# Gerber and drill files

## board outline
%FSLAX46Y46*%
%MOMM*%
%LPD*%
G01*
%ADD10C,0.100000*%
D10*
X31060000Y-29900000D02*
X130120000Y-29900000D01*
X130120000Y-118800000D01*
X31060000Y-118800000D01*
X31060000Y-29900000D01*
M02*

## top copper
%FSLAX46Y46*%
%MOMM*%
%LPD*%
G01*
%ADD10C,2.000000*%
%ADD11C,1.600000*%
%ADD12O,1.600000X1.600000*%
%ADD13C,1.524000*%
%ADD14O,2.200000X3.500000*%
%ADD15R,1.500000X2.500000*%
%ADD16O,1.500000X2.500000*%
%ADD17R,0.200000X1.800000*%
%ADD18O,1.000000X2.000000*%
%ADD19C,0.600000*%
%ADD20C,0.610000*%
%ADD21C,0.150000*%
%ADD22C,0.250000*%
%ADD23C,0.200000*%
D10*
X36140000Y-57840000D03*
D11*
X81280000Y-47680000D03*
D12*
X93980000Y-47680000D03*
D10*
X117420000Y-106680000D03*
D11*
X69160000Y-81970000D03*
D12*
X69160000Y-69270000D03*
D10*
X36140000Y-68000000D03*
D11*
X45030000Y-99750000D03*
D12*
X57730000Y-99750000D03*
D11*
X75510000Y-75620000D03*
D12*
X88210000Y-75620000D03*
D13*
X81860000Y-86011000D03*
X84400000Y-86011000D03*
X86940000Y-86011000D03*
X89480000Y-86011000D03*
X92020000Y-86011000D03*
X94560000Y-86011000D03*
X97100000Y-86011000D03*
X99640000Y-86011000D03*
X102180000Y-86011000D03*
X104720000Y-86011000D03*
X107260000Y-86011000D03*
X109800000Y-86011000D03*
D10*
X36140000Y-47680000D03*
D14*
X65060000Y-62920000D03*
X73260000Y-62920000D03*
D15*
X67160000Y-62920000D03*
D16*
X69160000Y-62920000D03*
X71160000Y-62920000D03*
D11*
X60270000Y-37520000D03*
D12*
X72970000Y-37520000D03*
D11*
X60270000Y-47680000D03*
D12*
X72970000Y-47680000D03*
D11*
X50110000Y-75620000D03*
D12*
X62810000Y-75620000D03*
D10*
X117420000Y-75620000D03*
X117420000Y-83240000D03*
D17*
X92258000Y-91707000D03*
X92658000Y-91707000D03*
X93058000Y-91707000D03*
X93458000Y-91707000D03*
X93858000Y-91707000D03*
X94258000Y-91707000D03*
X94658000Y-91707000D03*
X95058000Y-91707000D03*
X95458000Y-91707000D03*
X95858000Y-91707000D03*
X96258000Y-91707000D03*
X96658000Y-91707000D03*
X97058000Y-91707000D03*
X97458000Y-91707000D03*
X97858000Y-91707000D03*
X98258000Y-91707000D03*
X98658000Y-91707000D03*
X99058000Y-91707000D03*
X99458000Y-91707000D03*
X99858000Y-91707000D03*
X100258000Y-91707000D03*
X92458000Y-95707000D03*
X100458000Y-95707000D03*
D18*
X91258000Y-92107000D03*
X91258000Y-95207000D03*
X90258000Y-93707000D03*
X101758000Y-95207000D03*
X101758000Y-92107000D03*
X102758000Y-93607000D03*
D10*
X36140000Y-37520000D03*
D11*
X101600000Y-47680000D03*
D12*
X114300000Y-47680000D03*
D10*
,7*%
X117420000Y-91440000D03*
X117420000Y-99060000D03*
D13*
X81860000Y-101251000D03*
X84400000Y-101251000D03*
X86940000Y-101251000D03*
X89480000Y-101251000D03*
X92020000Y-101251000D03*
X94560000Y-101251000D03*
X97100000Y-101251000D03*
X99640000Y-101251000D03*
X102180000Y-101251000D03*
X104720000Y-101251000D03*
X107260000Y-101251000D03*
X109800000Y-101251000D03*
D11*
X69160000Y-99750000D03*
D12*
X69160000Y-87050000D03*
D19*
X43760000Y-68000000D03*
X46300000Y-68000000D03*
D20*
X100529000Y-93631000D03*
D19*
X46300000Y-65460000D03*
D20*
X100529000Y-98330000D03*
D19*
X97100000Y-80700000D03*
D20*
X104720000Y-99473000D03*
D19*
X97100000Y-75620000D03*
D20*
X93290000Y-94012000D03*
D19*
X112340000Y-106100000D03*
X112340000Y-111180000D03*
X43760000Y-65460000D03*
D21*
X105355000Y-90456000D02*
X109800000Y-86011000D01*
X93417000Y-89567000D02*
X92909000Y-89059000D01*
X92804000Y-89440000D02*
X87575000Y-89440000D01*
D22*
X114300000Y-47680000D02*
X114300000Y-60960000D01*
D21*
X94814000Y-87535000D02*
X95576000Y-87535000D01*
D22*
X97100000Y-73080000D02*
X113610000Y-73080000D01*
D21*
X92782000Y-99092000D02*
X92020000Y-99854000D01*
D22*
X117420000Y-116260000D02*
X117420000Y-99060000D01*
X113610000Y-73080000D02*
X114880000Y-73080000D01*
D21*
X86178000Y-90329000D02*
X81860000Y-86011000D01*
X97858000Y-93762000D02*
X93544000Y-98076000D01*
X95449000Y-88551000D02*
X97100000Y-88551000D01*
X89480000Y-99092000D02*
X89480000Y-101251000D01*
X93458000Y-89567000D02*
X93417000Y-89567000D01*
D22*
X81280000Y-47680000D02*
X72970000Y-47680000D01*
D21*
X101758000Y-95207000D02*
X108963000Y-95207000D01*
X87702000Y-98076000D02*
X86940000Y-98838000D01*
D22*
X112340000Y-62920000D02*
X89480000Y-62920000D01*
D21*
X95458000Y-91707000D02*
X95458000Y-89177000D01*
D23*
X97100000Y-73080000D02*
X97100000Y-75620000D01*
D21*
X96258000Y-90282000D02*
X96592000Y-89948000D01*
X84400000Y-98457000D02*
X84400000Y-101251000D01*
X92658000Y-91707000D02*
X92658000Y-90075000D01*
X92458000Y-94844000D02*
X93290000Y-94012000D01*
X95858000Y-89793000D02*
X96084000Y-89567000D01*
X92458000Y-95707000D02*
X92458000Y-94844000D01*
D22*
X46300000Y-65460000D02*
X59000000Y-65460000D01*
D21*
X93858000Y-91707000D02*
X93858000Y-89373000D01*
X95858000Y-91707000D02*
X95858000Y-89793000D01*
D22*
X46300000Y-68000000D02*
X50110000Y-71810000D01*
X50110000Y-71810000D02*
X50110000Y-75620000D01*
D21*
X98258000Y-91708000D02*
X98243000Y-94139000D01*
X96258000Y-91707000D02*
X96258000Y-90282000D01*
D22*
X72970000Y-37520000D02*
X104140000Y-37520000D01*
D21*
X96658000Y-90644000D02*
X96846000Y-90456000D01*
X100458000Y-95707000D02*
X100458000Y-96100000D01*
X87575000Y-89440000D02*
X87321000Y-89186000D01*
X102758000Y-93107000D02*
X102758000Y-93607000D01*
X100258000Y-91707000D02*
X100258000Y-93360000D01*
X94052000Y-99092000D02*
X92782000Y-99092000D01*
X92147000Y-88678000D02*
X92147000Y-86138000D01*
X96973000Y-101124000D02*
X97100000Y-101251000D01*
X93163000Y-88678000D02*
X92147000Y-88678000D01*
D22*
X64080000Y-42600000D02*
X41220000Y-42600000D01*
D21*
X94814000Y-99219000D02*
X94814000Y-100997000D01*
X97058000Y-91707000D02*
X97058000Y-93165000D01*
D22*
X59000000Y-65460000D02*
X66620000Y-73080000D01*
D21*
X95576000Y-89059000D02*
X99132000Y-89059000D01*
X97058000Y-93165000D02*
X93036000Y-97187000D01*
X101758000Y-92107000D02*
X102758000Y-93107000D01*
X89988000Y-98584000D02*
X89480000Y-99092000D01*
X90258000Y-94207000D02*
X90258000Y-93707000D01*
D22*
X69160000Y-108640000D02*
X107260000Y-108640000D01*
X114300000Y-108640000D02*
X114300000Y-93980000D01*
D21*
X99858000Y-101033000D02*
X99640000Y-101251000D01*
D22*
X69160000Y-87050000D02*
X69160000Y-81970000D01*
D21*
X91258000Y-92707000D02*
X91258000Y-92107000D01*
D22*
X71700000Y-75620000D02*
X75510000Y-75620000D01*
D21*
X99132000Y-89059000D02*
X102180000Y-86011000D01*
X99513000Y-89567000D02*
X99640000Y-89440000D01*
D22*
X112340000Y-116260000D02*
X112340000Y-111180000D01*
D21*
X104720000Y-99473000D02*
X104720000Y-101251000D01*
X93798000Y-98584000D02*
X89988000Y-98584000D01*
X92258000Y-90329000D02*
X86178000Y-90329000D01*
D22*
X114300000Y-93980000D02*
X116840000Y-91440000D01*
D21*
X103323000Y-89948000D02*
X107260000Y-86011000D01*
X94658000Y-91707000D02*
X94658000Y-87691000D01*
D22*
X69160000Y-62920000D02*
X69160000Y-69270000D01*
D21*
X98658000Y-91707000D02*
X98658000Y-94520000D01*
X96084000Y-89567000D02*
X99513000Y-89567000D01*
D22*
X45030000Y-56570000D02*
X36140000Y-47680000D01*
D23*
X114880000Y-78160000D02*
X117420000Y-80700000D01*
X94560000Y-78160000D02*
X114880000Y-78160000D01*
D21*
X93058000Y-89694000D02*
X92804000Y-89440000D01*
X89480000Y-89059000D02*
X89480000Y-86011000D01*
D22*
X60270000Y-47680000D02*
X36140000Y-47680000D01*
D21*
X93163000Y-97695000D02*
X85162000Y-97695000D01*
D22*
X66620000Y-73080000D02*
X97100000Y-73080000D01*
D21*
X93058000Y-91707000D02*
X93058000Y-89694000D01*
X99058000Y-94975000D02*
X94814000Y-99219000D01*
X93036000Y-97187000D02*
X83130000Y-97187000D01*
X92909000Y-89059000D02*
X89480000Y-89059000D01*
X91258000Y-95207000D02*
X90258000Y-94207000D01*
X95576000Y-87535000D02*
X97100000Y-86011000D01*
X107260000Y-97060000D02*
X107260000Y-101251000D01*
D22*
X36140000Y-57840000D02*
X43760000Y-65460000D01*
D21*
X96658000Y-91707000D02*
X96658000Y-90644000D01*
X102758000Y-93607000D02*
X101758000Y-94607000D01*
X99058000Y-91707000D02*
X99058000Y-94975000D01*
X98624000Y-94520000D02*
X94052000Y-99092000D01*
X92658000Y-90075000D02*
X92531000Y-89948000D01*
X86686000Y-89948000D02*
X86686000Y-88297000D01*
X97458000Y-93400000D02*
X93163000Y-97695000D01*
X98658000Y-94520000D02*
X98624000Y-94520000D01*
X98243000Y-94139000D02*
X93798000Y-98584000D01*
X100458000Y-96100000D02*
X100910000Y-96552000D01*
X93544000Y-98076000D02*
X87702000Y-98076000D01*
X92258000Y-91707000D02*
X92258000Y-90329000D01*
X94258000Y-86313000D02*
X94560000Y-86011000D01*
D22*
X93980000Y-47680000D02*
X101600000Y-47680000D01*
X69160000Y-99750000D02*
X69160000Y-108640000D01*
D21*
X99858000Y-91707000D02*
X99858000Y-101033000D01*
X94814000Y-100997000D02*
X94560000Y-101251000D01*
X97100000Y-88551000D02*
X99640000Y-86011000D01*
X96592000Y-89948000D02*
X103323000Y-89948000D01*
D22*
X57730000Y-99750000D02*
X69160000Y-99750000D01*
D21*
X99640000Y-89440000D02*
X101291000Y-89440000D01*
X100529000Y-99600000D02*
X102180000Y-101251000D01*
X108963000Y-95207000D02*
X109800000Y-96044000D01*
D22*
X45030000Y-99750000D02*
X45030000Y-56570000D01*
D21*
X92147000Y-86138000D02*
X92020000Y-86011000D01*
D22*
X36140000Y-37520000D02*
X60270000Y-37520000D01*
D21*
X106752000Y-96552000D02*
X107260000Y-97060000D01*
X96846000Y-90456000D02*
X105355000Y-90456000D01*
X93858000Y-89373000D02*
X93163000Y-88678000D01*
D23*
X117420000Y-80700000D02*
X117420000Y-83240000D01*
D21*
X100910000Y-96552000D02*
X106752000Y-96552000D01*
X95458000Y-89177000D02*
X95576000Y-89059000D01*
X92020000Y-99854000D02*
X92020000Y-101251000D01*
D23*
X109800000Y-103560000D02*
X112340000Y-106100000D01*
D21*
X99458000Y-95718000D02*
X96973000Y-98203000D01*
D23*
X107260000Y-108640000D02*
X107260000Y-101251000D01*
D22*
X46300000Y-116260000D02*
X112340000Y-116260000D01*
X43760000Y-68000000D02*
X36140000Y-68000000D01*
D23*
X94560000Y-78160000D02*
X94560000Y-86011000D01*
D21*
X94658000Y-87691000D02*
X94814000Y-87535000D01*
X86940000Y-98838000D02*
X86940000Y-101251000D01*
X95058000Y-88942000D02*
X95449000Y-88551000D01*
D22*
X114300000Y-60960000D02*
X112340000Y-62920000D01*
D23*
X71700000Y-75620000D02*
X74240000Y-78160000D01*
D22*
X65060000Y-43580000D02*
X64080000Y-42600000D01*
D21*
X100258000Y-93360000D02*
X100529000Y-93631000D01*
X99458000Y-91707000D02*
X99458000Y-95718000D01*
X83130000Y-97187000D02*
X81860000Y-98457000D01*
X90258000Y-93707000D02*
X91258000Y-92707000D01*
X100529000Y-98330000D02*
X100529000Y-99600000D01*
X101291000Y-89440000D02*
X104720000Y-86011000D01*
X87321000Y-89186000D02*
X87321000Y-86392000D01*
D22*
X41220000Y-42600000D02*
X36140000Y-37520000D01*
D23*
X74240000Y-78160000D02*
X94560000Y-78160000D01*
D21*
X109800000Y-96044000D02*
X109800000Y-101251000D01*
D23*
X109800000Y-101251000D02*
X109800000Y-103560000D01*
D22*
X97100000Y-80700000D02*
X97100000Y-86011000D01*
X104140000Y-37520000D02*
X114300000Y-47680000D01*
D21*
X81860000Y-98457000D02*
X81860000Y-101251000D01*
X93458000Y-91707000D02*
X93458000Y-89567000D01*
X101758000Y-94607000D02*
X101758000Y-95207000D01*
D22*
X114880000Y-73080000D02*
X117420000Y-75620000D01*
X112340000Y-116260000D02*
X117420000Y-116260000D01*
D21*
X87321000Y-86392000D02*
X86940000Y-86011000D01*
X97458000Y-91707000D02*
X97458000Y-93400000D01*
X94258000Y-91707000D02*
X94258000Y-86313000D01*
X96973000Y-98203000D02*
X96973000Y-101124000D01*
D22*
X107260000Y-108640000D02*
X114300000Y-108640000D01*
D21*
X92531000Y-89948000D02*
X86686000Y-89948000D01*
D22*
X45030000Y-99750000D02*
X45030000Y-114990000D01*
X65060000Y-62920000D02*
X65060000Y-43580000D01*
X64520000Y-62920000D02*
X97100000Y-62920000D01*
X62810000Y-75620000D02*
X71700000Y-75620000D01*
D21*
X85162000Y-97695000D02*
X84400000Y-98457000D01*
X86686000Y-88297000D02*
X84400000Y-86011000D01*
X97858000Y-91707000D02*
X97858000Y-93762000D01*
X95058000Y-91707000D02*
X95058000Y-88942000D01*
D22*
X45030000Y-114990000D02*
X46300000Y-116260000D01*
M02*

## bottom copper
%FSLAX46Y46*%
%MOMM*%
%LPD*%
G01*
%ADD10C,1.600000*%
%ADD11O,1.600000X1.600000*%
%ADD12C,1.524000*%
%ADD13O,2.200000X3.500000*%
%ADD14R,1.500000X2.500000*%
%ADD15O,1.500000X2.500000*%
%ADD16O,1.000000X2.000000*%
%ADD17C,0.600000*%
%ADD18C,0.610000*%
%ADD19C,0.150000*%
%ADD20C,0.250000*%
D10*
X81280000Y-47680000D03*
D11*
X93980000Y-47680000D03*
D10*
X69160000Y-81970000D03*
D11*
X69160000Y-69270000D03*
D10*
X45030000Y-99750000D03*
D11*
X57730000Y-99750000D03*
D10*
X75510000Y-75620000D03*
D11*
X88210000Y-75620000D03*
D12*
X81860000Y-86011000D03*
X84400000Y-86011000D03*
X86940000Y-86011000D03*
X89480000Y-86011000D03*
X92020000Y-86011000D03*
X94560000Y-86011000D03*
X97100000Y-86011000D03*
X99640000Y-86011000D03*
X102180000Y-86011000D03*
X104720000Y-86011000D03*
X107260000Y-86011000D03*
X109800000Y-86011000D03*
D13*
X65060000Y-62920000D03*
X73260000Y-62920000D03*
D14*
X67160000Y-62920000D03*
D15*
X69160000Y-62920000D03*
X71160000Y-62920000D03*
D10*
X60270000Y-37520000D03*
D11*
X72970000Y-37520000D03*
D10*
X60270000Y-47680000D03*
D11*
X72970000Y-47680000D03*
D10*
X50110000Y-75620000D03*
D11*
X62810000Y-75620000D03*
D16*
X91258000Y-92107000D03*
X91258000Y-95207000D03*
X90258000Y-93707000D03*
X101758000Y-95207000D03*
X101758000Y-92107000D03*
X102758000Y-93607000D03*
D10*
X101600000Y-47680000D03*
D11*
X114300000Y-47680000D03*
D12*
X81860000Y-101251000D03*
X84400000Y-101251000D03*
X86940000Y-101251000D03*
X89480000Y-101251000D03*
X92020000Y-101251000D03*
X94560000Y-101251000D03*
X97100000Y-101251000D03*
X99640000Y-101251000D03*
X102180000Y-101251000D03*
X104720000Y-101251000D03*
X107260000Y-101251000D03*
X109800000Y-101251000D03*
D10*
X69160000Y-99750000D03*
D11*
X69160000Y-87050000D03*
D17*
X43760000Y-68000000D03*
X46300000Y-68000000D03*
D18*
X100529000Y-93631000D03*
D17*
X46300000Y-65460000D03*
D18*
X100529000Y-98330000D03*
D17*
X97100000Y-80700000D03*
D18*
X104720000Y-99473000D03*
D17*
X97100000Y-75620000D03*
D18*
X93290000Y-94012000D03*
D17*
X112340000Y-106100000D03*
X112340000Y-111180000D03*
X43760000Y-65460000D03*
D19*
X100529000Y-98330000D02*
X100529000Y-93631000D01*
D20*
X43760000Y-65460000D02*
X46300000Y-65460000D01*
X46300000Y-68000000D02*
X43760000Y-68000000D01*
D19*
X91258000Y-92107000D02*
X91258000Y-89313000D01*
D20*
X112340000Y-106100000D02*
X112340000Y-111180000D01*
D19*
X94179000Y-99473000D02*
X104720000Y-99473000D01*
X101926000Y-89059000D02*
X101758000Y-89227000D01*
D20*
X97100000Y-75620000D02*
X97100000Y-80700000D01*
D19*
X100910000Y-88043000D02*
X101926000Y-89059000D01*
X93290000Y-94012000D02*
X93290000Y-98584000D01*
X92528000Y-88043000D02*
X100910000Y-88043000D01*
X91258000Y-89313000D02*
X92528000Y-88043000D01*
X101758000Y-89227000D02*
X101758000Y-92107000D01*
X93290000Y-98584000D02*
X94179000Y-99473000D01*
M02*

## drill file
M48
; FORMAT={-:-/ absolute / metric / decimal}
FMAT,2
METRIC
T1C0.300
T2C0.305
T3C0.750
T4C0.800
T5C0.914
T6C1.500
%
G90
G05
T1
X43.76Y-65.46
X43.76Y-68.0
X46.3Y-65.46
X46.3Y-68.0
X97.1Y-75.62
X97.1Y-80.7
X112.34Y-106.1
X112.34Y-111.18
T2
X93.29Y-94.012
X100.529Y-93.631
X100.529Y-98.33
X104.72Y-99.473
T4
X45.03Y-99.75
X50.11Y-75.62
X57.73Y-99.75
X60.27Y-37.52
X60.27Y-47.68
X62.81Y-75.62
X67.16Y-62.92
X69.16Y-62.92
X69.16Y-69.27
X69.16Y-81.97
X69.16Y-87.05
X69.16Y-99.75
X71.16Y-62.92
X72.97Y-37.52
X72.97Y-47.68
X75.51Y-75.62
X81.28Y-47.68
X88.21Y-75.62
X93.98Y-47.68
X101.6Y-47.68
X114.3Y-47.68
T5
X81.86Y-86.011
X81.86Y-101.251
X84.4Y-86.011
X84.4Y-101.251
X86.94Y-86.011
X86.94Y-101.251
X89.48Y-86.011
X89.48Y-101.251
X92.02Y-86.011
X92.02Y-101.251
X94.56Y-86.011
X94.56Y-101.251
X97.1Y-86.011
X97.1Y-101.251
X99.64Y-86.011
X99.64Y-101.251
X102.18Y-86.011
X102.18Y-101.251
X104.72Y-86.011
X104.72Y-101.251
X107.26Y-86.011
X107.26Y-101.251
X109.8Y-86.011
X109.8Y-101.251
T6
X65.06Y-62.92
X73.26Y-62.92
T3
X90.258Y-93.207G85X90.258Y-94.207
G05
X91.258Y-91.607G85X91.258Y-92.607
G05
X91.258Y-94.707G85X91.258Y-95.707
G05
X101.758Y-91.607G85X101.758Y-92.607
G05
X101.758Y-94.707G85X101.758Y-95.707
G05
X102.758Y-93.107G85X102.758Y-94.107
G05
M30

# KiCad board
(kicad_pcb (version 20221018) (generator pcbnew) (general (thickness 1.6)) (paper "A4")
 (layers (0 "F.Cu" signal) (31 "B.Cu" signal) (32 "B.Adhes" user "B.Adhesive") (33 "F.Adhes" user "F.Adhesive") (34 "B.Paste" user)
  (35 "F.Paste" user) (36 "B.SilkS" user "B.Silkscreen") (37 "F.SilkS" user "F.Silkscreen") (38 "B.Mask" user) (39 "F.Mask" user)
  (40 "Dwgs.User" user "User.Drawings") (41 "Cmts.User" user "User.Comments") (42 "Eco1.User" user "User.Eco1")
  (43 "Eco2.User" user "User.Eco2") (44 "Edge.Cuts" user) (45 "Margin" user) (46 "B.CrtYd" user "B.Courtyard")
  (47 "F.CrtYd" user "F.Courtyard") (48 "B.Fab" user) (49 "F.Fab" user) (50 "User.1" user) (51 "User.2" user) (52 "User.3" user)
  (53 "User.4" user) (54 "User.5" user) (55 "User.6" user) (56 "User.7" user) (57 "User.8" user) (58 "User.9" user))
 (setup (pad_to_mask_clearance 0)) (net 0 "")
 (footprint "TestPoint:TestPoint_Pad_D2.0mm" (layer "F.Cu") (at 36.14 57.84)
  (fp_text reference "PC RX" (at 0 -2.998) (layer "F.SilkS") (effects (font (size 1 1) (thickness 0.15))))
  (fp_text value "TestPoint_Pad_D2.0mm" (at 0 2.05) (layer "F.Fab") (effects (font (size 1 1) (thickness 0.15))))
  (pad "3" smd circle (at 0 0) (size 2 2) (layers "F.Cu" "F.Mask")))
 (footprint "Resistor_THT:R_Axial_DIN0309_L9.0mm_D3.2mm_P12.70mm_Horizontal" (layer "F.Cu") (at 81.28 47.68)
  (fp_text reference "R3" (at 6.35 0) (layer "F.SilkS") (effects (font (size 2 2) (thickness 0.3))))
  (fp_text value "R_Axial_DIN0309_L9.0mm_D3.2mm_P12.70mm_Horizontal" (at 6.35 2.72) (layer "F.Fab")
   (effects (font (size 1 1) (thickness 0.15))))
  (pad "1" thru_hole circle (at 0 0) (size 1.6 1.6) (drill 0.8) (layers "*.Cu" "*.Mask"))
  (pad "2" thru_hole oval (at 12.7 0) (size 1.6 1.6) (drill 0.8) (layers "*.Cu" "*.Mask")))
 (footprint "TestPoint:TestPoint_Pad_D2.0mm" (layer "F.Cu") (at 117.42 106.68)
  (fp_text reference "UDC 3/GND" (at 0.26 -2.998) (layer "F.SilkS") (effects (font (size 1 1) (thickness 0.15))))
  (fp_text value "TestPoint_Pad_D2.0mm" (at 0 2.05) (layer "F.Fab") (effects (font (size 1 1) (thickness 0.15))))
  (pad "9" smd circle (at 0 0) (size 2 2) (layers "F.Cu" "F.Mask")))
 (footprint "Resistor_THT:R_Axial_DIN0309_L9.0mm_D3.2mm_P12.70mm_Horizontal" (layer "F.Cu") (at 69.16 81.97 90)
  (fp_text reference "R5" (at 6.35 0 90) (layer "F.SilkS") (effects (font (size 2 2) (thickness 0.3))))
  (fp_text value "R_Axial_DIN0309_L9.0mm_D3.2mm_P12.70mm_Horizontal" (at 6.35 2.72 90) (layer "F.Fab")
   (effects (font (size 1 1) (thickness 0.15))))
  (pad "1" thru_hole circle (at 0 0 90) (size 1.6 1.6) (drill 0.8) (layers "*.Cu" "*.Mask"))
  (pad "2" thru_hole oval (at 12.7 0 90) (size 1.6 1.6) (drill 0.8) (layers "*.Cu" "*.Mask")))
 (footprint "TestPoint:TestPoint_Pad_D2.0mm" (layer "F.Cu") (at 36.14 68)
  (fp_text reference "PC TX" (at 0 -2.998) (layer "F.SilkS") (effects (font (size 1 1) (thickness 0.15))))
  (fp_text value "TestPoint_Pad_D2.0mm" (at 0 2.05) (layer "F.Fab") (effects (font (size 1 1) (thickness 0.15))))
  (pad "4" smd circle (at 0 0) (size 2 2) (layers "F.Cu" "F.Mask")))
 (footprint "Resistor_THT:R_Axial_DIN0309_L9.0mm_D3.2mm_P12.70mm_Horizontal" (layer "F.Cu") (at 45.03 99.75)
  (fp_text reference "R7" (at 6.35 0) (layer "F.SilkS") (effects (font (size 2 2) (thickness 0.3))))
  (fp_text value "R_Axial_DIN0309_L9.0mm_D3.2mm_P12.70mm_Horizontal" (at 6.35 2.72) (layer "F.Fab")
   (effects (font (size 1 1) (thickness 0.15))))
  (pad "1" thru_hole circle (at 0 0) (size 1.6 1.6) (drill 0.8) (layers "*.Cu" "*.Mask"))
  (pad "2" thru_hole oval (at 12.7 0) (size 1.6 1.6) (drill 0.8) (layers "*.Cu" "*.Mask")))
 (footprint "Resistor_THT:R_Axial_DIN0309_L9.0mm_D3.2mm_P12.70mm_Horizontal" (layer "F.Cu") (at 75.51 75.62)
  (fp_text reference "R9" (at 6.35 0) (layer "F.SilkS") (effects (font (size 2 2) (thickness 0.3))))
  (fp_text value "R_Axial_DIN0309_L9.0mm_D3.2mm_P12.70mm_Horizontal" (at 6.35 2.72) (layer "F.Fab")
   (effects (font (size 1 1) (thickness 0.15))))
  (pad "1" thru_hole circle (at 0 0) (size 1.6 1.6) (drill 0.8) (layers "*.Cu" "*.Mask"))
  (pad "2" thru_hole oval (at 12.7 0) (size 1.6 1.6) (drill 0.8) (layers "*.Cu" "*.Mask")))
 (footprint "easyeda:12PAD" (layer "F.Cu") (at 81.86 86.011)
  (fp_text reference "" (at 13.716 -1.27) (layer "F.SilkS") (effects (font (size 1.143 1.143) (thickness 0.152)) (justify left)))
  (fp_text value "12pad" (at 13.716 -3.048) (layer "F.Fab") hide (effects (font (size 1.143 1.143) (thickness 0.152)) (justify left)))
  (pad "1" thru_hole circle (at 0 0) (size 1.524 1.524) (drill 0.914) (layers "*.Cu" "*.Paste" "*.Mask"))
  (pad "2" thru_hole circle (at 2.54 0) (size 1.524 1.524) (drill 0.914) (layers "*.Cu" "*.Paste" "*.Mask"))
  (pad "3" thru_hole circle (at 5.08 0) (size 1.524 1.524) (drill 0.914) (layers "*.Cu" "*.Paste" "*.Mask"))
  (pad "4" thru_hole circle (at 7.62 0) (size 1.524 1.524) (drill 0.914) (layers "*.Cu" "*.Paste" "*.Mask"))
  (pad "5" thru_hole circle (at 10.16 0) (size 1.524 1.524) (drill 0.914) (layers "*.Cu" "*.Paste" "*.Mask"))
  (pad "6" thru_hole circle (at 12.7 0) (size 1.524 1.524) (drill 0.914) (layers "*.Cu" "*.Paste" "*.Mask"))
  (pad "7" thru_hole circle (at 15.24 0) (size 1.524 1.524) (drill 0.914) (layers "*.Cu" "*.Paste" "*.Mask"))
  (pad "8" thru_hole circle (at 17.78 0) (size 1.524 1.524) (drill 0.914) (layers "*.Cu" "*.Paste" "*.Mask"))
  (pad "9" thru_hole circle (at 20.32 0) (size 1.524 1.524) (drill 0.914) (layers "*.Cu" "*.Paste" "*.Mask"))
  (pad "10" thru_hole circle (at 22.86 0) (size 1.524 1.524) (drill 0.914) (layers "*.Cu" "*.Paste" "*.Mask"))
  (pad "11" thru_hole circle (at 25.4 0) (size 1.524 1.524) (drill 0.914) (layers "*.Cu" "*.Paste" "*.Mask"))
  (pad "12" thru_hole circle (at 27.94 0) (size 1.524 1.524) (drill 0.914) (layers "*.Cu" "*.Paste" "*.Mask")))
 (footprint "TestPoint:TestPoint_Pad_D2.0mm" (layer "F.Cu") (at 36.14 47.68)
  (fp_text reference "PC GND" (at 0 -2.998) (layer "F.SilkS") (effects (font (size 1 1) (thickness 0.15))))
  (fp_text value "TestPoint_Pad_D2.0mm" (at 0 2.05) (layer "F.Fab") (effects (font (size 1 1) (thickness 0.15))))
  (pad "2" smd circle (at 0 0) (size 2 2) (layers "F.Cu" "F.Mask")))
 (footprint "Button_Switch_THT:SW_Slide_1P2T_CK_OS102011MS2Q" (layer "F.Cu") (at 67.16 62.92)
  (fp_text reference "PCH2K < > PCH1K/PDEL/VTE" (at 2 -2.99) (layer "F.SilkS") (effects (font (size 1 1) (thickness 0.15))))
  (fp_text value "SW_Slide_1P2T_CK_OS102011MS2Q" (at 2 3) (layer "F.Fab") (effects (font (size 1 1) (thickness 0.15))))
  (pad "" thru_hole oval (at -2.1 0) (size 2.2 3.5) (drill 1.5) (layers "*.Cu" "*.Mask"))
  (pad "" thru_hole oval (at 6.1 0) (size 2.2 3.5) (drill 1.5) (layers "*.Cu" "*.Mask"))
  (pad "1" thru_hole rect (at 0 0) (size 1.5 2.5) (drill 0.8) (layers "*.Cu" "*.Mask"))
  (pad "2" thru_hole oval (at 2 0) (size 1.5 2.5) (drill 0.8) (layers "*.Cu" "*.Mask"))
  (pad "3" thru_hole oval (at 4 0) (size 1.5 2.5) (drill 0.8) (layers "*.Cu" "*.Mask")))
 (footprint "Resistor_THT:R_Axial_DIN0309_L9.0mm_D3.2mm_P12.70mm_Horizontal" (layer "F.Cu") (at 60.27 37.52)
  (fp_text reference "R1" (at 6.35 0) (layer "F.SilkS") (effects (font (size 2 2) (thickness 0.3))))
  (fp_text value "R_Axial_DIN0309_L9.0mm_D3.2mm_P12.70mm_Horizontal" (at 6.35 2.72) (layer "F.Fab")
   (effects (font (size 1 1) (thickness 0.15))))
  (pad "1" thru_hole circle (at 0 0) (size 1.6 1.6) (drill 0.8) (layers "*.Cu" "*.Mask"))
  (pad "2" thru_hole oval (at 12.7 0) (size 1.6 1.6) (drill 0.8) (layers "*.Cu" "*.Mask")))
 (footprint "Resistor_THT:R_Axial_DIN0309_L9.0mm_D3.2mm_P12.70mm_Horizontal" (layer "F.Cu") (at 60.27 47.68)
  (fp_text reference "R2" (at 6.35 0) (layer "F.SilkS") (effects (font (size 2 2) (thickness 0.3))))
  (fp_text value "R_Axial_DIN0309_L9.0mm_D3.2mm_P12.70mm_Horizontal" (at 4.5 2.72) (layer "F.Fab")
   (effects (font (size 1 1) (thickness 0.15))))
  (pad "1" thru_hole circle (at 0 0) (size 1.6 1.6) (drill 0.8) (layers "*.Cu" "*.Mask"))
  (pad "2" thru_hole oval (at 12.7 0) (size 1.6 1.6) (drill 0.8) (layers "*.Cu" "*.Mask")))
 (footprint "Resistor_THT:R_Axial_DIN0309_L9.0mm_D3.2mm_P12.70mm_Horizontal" (layer "F.Cu") (at 50.11 75.62)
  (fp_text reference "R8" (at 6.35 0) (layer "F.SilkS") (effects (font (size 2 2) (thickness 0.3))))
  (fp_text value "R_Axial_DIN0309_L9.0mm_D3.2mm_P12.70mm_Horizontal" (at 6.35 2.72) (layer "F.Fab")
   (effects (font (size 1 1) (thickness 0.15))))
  (pad "1" thru_hole circle (at 0 0) (size 1.6 1.6) (drill 0.8) (layers "*.Cu" "*.Mask"))
  (pad "2" thru_hole oval (at 12.7 0) (size 1.6 1.6) (drill 0.8) (layers "*.Cu" "*.Mask")))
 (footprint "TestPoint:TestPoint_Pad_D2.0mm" (layer "F.Cu") (at 117.42 75.62)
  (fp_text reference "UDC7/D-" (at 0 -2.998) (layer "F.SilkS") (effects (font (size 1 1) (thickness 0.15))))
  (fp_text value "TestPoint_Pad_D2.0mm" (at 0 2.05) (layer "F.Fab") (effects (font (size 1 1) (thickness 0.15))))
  (pad "5" smd circle (at 0 0) (size 2 2) (layers "F.Cu" "F.Mask")))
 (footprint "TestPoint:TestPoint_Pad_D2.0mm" (layer "F.Cu") (at 117.42 83.24)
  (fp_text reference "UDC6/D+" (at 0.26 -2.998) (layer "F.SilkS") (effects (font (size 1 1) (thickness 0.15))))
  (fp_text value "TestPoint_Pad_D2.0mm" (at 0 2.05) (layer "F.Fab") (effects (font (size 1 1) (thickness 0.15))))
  (pad "6" smd circle (at 0 0) (size 2 2) (layers "F.Cu" "F.Mask")))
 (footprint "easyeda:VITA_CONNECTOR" (layer "F.Cu") (at 91.258 92.107)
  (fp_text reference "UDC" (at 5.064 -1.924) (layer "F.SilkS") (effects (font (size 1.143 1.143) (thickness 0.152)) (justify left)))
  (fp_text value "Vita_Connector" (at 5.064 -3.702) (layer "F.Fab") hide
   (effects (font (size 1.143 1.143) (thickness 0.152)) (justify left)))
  (pad "1" smd rect (at 1 -0.4) (size 0.2 1.8) (layers "F.Cu" "F.Paste" "F.Mask"))
  (pad "2" smd rect (at 1.4 -0.4) (size 0.2 1.8) (layers "F.Cu" "F.Paste" "F.Mask"))
  (pad "3" smd rect (at 1.8 -0.4) (size 0.2 1.8) (layers "F.Cu" "F.Paste" "F.Mask"))
  (pad "4" smd rect (at 2.2 -0.4) (size 0.2 1.8) (layers "F.Cu" "F.Paste" "F.Mask"))
  (pad "5" smd rect (at 2.6 -0.4) (size 0.2 1.8) (layers "F.Cu" "F.Paste" "F.Mask"))
  (pad "6" smd rect (at 3 -0.4) (size 0.2 1.8) (layers "F.Cu" "F.Paste" "F.Mask"))
  (pad "7" smd rect (at 3.4 -0.4) (size 0.2 1.8) (layers "F.Cu" "F.Paste" "F.Mask"))
  (pad "8" smd rect (at 3.8 -0.4) (size 0.2 1.8) (layers "F.Cu" "F.Paste" "F.Mask"))
  (pad "9" smd rect (at 4.2 -0.4) (size 0.2 1.8) (layers "F.Cu" "F.Paste" "F.Mask"))
  (pad "10" smd rect (at 4.6 -0.4) (size 0.2 1.8) (layers "F.Cu" "F.Paste" "F.Mask"))
  (pad "11" smd rect (at 5 -0.4) (size 0.2 1.8) (layers "F.Cu" "F.Paste" "F.Mask"))
  (pad "12" smd rect (at 5.4 -0.4) (size 0.2 1.8) (layers "F.Cu" "F.Paste" "F.Mask"))
  (pad "13" smd rect (at 5.8 -0.4) (size 0.2 1.8) (layers "F.Cu" "F.Paste" "F.Mask"))
  (pad "14" smd rect (at 6.2 -0.4) (size 0.2 1.8) (layers "F.Cu" "F.Paste" "F.Mask"))
  (pad "15" smd rect (at 6.6 -0.4) (size 0.2 1.8) (layers "F.Cu" "F.Paste" "F.Mask"))
  (pad "16" smd rect (at 7 -0.4) (size 0.2 1.8) (layers "F.Cu" "F.Paste" "F.Mask"))
  (pad "17" smd rect (at 7.4 -0.4) (size 0.2 1.8) (layers "F.Cu" "F.Paste" "F.Mask"))
  (pad "18" smd rect (at 7.8 -0.4) (size 0.2 1.8) (layers "F.Cu" "F.Paste" "F.Mask"))
  (pad "19" smd rect (at 8.2 -0.4) (size 0.2 1.8) (layers "F.Cu" "F.Paste" "F.Mask"))
  (pad "20" smd rect (at 8.6 -0.4) (size 0.2 1.8) (layers "F.Cu" "F.Paste" "F.Mask"))
  (pad "21" smd rect (at 9 -0.4) (size 0.2 1.8) (layers "F.Cu" "F.Paste" "F.Mask"))
  (pad "22" smd rect (at 1.2 3.6) (size 0.2 1.8) (layers "F.Cu" "F.Paste" "F.Mask"))
  (pad "23" smd rect (at 9.2 3.6) (size 0.2 1.8) (layers "F.Cu" "F.Paste" "F.Mask"))
  (pad "24" thru_hole oval (at 0 0) (size 1 2) (drill oval 0.75 1.75) (layers "*.Cu" "*.Paste" "*.Mask"))
  (pad "25" thru_hole oval (at 0 3.1) (size 1 2) (drill oval 0.75 1.75) (layers "*.Cu" "*.Paste" "*.Mask"))
  (pad "26" thru_hole oval (at -1 1.6) (size 1 2) (drill oval 0.75 1.75) (layers "*.Cu" "*.Paste" "*.Mask"))
  (pad "27" thru_hole oval (at 10.5 3.1) (size 1 2) (drill oval 0.75 1.75) (layers "*.Cu" "*.Paste" "*.Mask"))
  (pad "28" thru_hole oval (at 10.5 0) (size 1 2) (drill oval 0.75 1.75) (layers "*.Cu" "*.Paste" "*.Mask"))
  (pad "29" thru_hole oval (at 11.5 1.5) (size 1 2) (drill oval 0.75 1.75) (layers "*.Cu" "*.Paste" "*.Mask")))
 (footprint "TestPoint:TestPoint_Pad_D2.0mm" (layer "F.Cu") (at 36.14 37.52)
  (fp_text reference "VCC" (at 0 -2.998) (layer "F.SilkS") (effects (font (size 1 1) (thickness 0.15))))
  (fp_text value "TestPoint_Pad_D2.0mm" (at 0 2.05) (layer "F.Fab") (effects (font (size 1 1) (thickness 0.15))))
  (pad "1" smd circle (at 0 0) (size 2 2) (layers "F.Cu" "F.Mask")))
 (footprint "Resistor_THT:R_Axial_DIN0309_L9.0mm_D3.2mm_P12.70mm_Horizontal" (layer "F.Cu") (at 101.6 47.68)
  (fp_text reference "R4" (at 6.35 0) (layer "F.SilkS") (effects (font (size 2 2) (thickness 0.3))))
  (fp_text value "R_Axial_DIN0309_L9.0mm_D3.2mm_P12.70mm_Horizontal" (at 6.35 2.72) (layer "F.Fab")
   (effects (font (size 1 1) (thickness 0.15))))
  (pad "1" thru_hole circle (at 0 0) (size 1.6 1.6) (drill 0.8) (layers "*.Cu" "*.Mask"))
  (pad "2" thru_hole oval (at 12.7 0) (size 1.6 1.6) (drill 0.8) (layers "*.Cu" "*.Mask")))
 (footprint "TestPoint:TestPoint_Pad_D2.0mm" (layer "F.Cu") (at 117.42 91.44)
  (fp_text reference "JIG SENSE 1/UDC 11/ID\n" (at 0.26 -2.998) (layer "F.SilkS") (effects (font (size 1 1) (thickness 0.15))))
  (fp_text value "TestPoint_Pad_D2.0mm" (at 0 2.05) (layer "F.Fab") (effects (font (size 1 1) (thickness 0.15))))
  (pad "7" smd circle (at 0 0) (size 2 2) (layers "F.Cu" "F.Mask")))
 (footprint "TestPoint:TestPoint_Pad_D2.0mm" (layer "F.Cu") (at 117.42 99.06)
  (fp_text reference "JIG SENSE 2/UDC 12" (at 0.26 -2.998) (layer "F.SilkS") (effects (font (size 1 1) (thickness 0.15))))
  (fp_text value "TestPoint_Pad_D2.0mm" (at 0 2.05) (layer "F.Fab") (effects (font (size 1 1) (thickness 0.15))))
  (pad "8" smd circle (at 0 0) (size 2 2) (layers "F.Cu" "F.Mask")))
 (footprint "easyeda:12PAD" (layer "F.Cu") (at 81.86 101.251)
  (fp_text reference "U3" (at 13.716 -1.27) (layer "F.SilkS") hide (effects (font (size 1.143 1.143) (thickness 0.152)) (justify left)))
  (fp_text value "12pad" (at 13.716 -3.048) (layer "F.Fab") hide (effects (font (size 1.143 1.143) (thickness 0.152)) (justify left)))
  (pad "1" thru_hole circle (at 0 0) (size 1.524 1.524) (drill 0.914) (layers "*.Cu" "*.Paste" "*.Mask"))
  (pad "2" thru_hole circle (at 2.54 0) (size 1.524 1.524) (drill 0.914) (layers "*.Cu" "*.Paste" "*.Mask"))
  (pad "3" thru_hole circle (at 5.08 0) (size 1.524 1.524) (drill 0.914) (layers "*.Cu" "*.Paste" "*.Mask"))
  (pad "4" thru_hole circle (at 7.62 0) (size 1.524 1.524) (drill 0.914) (layers "*.Cu" "*.Paste" "*.Mask"))
  (pad "5" thru_hole circle (at 10.16 0) (size 1.524 1.524) (drill 0.914) (layers "*.Cu" "*.Paste" "*.Mask"))
  (pad "6" thru_hole circle (at 12.7 0) (size 1.524 1.524) (drill 0.914) (layers "*.Cu" "*.Paste" "*.Mask"))
  (pad "7" thru_hole circle (at 15.24 0) (size 1.524 1.524) (drill 0.914) (layers "*.Cu" "*.Paste" "*.Mask"))
  (pad "8" thru_hole circle (at 17.78 0) (size 1.524 1.524) (drill 0.914) (layers "*.Cu" "*.Paste" "*.Mask"))
  (pad "9" thru_hole circle (at 20.32 0) (size 1.524 1.524) (drill 0.914) (layers "*.Cu" "*.Paste" "*.Mask"))
  (pad "10" thru_hole circle (at 22.86 0) (size 1.524 1.524) (drill 0.914) (layers "*.Cu" "*.Paste" "*.Mask"))
  (pad "11" thru_hole circle (at 25.4 0) (size 1.524 1.524) (drill 0.914) (layers "*.Cu" "*.Paste" "*.Mask"))
  (pad "12" thru_hole circle (at 27.94 0) (size 1.524 1.524) (drill 0.914) (layers "*.Cu" "*.Paste" "*.Mask")))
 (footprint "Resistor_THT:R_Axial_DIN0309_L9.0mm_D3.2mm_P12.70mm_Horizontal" (layer "F.Cu") (at 69.16 99.75 90)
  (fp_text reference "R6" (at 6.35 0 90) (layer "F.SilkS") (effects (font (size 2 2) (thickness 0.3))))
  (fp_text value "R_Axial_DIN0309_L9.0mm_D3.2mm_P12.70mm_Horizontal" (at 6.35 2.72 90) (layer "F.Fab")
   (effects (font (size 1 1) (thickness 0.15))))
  (pad "1" thru_hole circle (at 0 0 90) (size 1.6 1.6) (drill 0.8) (layers "*.Cu" "*.Mask"))
  (pad "2" thru_hole oval (at 12.7 0 90) (size 1.6 1.6) (drill 0.8) (layers "*.Cu" "*.Mask")))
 (gr_rect (start 31.06 29.9) (end 130.12 118.8) (stroke (width 0.1) (type default)) (fill none) (layer "Edge.Cuts"))
 (segment (start 105.355 90.456) (end 109.8 86.011) (width 0.15) (layer "F.Cu") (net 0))
 (segment (start 93.417 89.567) (end 92.909 89.059) (width 0.15) (layer "F.Cu") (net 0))
 (segment (start 92.804 89.44) (end 87.575 89.44) (width 0.15) (layer "F.Cu") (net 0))
 (segment (start 114.3 47.68) (end 114.3 60.96) (width 0.25) (layer "F.Cu") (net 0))
 (segment (start 94.814 87.535) (end 95.576 87.535) (width 0.15) (layer "F.Cu") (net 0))
 (segment (start 97.1 73.08) (end 113.61 73.08) (width 0.25) (layer "F.Cu") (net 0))
 (segment (start 92.782 99.092) (end 92.02 99.854) (width 0.15) (layer "F.Cu") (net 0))
 (segment (start 117.42 116.26) (end 117.42 99.06) (width 0.25) (layer "F.Cu") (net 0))
 (segment (start 113.61 73.08) (end 114.88 73.08) (width 0.25) (layer "F.Cu") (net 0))
 (segment (start 86.178 90.329) (end 81.86 86.011) (width 0.15) (layer "F.Cu") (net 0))
 (segment (start 97.858 93.762) (end 93.544 98.076) (width 0.15) (layer "F.Cu") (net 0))
 (segment (start 95.449 88.551) (end 97.1 88.551) (width 0.15) (layer "F.Cu") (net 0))
 (segment (start 89.48 99.092) (end 89.48 101.251) (width 0.15) (layer "F.Cu") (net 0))
 (segment (start 93.458 89.567) (end 93.417 89.567) (width 0.15) (layer "F.Cu") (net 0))
 (segment (start 81.28 47.68) (end 72.97 47.68) (width 0.25) (layer "F.Cu") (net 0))
 (segment (start 101.758 95.207) (end 108.963 95.207) (width 0.15) (layer "F.Cu") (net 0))
 (segment (start 87.702 98.076) (end 86.94 98.838) (width 0.15) (layer "F.Cu") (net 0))
 (segment (start 112.34 62.92) (end 89.48 62.92) (width 0.25) (layer "F.Cu") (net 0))
 (segment (start 95.458 91.707) (end 95.458 89.177) (width 0.15) (layer "F.Cu") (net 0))
 (segment (start 97.1 73.08) (end 97.1 75.62) (width 0.2) (layer "F.Cu") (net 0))
 (segment (start 96.258 90.282) (end 96.592 89.948) (width 0.15) (layer "F.Cu") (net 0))
 (segment (start 84.4 98.457) (end 84.4 101.251) (width 0.15) (layer "F.Cu") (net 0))
 (segment (start 92.658 91.707) (end 92.658 90.075) (width 0.15) (layer "F.Cu") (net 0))
 (segment (start 92.458 94.844) (end 93.29 94.012) (width 0.15) (layer "F.Cu") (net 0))
 (segment (start 95.858 89.793) (end 96.084 89.567) (width 0.15) (layer "F.Cu") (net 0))
 (segment (start 92.458 95.707) (end 92.458 94.844) (width 0.15) (layer "F.Cu") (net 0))
 (segment (start 46.3 65.46) (end 59 65.46) (width 0.25) (layer "F.Cu") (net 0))
 (segment (start 93.858 91.707) (end 93.858 89.373) (width 0.15) (layer "F.Cu") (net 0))
 (segment (start 95.858 91.707) (end 95.858 89.793) (width 0.15) (layer "F.Cu") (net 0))
 (segment (start 46.3 68) (end 50.11 71.81) (width 0.25) (layer "F.Cu") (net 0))
 (segment (start 50.11 71.81) (end 50.11 75.62) (width 0.25) (layer "F.Cu") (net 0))
 (segment (start 98.258 91.708) (end 98.243 94.139) (width 0.15) (layer "F.Cu") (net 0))
 (segment (start 96.258 91.707) (end 96.258 90.282) (width 0.15) (layer "F.Cu") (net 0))
 (segment (start 72.97 37.52) (end 104.14 37.52) (width 0.25) (layer "F.Cu") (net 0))
 (segment (start 96.658 90.644) (end 96.846 90.456) (width 0.15) (layer "F.Cu") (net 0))
 (segment (start 100.458 95.707) (end 100.458 96.1) (width 0.15) (layer "F.Cu") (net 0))
 (segment (start 87.575 89.44) (end 87.321 89.186) (width 0.15) (layer "F.Cu") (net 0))
 (segment (start 102.758 93.107) (end 102.758 93.607) (width 0.15) (layer "F.Cu") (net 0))
 (segment (start 100.258 91.707) (end 100.258 93.36) (width 0.15) (layer "F.Cu") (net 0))
 (segment (start 94.052 99.092) (end 92.782 99.092) (width 0.15) (layer "F.Cu") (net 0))
 (segment (start 92.147 88.678) (end 92.147 86.138) (width 0.15) (layer "F.Cu") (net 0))
 (segment (start 96.973 101.124) (end 97.1 101.251) (width 0.15) (layer "F.Cu") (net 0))
 (segment (start 93.163 88.678) (end 92.147 88.678) (width 0.15) (layer "F.Cu") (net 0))
 (segment (start 64.08 42.6) (end 41.22 42.6) (width 0.25) (layer "F.Cu") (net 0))
 (segment (start 94.814 99.219) (end 94.814 100.997) (width 0.15) (layer "F.Cu") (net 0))
 (segment (start 97.058 91.707) (end 97.058 93.165) (width 0.15) (layer "F.Cu") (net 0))
 (segment (start 59 65.46) (end 66.62 73.08) (width 0.25) (layer "F.Cu") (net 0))
 (segment (start 95.576 89.059) (end 99.132 89.059) (width 0.15) (layer "F.Cu") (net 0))
 (segment (start 97.058 93.165) (end 93.036 97.187) (width 0.15) (layer "F.Cu") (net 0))
 (segment (start 101.758 92.107) (end 102.758 93.107) (width 0.15) (layer "F.Cu") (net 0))
 (segment (start 89.988 98.584) (end 89.48 99.092) (width 0.15) (layer "F.Cu") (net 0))
 (segment (start 90.258 94.207) (end 90.258 93.707) (width 0.15) (layer "F.Cu") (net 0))
 (segment (start 69.16 108.64) (end 107.26 108.64) (width 0.25) (layer "F.Cu") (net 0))
 (segment (start 114.3 108.64) (end 114.3 93.98) (width 0.25) (layer "F.Cu") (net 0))
 (segment (start 99.858 101.033) (end 99.64 101.251) (width 0.15) (layer "F.Cu") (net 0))
 (segment (start 69.16 87.05) (end 69.16 81.97) (width 0.25) (layer "F.Cu") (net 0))
 (segment (start 91.258 92.707) (end 91.258 92.107) (width 0.15) (layer "F.Cu") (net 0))
 (segment (start 71.7 75.62) (end 75.51 75.62) (width 0.25) (layer "F.Cu") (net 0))
 (segment (start 99.132 89.059) (end 102.18 86.011) (width 0.15) (layer "F.Cu") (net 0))
 (segment (start 99.513 89.567) (end 99.64 89.44) (width 0.15) (layer "F.Cu") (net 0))
 (segment (start 112.34 116.26) (end 112.34 111.18) (width 0.25) (layer "F.Cu") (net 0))
 (segment (start 104.72 99.473) (end 104.72 101.251) (width 0.15) (layer "F.Cu") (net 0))
 (segment (start 93.798 98.584) (end 89.988 98.584) (width 0.15) (layer "F.Cu") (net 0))
 (segment (start 92.258 90.329) (end 86.178 90.329) (width 0.15) (layer "F.Cu") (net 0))
 (segment (start 114.3 93.98) (end 116.84 91.44) (width 0.25) (layer "F.Cu") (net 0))
 (segment (start 103.323 89.948) (end 107.26 86.011) (width 0.15) (layer "F.Cu") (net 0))
 (segment (start 94.658 91.707) (end 94.658 87.691) (width 0.15) (layer "F.Cu") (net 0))
 (segment (start 69.16 62.92) (end 69.16 69.27) (width 0.25) (layer "F.Cu") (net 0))
 (segment (start 98.658 91.707) (end 98.658 94.52) (width 0.15) (layer "F.Cu") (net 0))
 (segment (start 96.084 89.567) (end 99.513 89.567) (width 0.15) (layer "F.Cu") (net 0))
 (segment (start 45.03 56.57) (end 36.14 47.68) (width 0.25) (layer "F.Cu") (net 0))
 (segment (start 114.88 78.16) (end 117.42 80.7) (width 0.2) (layer "F.Cu") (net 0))
 (segment (start 94.56 78.16) (end 114.88 78.16) (width 0.2) (layer "F.Cu") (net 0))
 (segment (start 93.058 89.694) (end 92.804 89.44) (width 0.15) (layer "F.Cu") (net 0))
 (segment (start 89.48 89.059) (end 89.48 86.011) (width 0.15) (layer "F.Cu") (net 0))
 (segment (start 60.27 47.68) (end 36.14 47.68) (width 0.25) (layer "F.Cu") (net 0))
 (segment (start 93.163 97.695) (end 85.162 97.695) (width 0.15) (layer "F.Cu") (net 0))
 (segment (start 66.62 73.08) (end 97.1 73.08) (width 0.25) (layer "F.Cu") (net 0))
 (segment (start 93.058 91.707) (end 93.058 89.694) (width 0.15) (layer "F.Cu") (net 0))
 (segment (start 99.058 94.975) (end 94.814 99.219) (width 0.15) (layer "F.Cu") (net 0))
 (segment (start 93.036 97.187) (end 83.13 97.187) (width 0.15) (layer "F.Cu") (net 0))
 (segment (start 92.909 89.059) (end 89.48 89.059) (width 0.15) (layer "F.Cu") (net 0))
 (segment (start 91.258 95.207) (end 90.258 94.207) (width 0.15) (layer "F.Cu") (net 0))
 (segment (start 95.576 87.535) (end 97.1 86.011) (width 0.15) (layer "F.Cu") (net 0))
 (segment (start 107.26 97.06) (end 107.26 101.251) (width 0.15) (layer "F.Cu") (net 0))
 (segment (start 36.14 57.84) (end 43.76 65.46) (width 0.25) (layer "F.Cu") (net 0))
 (segment (start 96.658 91.707) (end 96.658 90.644) (width 0.15) (layer "F.Cu") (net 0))
 (segment (start 102.758 93.607) (end 101.758 94.607) (width 0.15) (layer "F.Cu") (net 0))
 (segment (start 99.058 91.707) (end 99.058 94.975) (width 0.15) (layer "F.Cu") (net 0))
 (segment (start 98.624 94.52) (end 94.052 99.092) (width 0.15) (layer "F.Cu") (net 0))
 (segment (start 92.658 90.075) (end 92.531 89.948) (width 0.15) (layer "F.Cu") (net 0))
 (segment (start 86.686 89.948) (end 86.686 88.297) (width 0.15) (layer "F.Cu") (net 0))
 (segment (start 97.458 93.4) (end 93.163 97.695) (width 0.15) (layer "F.Cu") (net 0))
 (segment (start 98.658 94.52) (end 98.624 94.52) (width 0.15) (layer "F.Cu") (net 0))
 (segment (start 98.243 94.139) (end 93.798 98.584) (width 0.15) (layer "F.Cu") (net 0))
 (segment (start 100.458 96.1) (end 100.91 96.552) (width 0.15) (layer "F.Cu") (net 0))
 (segment (start 93.544 98.076) (end 87.702 98.076) (width 0.15) (layer "F.Cu") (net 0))
 (segment (start 92.258 91.707) (end 92.258 90.329) (width 0.15) (layer "F.Cu") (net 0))
 (segment (start 94.258 86.313) (end 94.56 86.011) (width 0.15) (layer "F.Cu") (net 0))
 (segment (start 93.98 47.68) (end 101.6 47.68) (width 0.25) (layer "F.Cu") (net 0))
 (segment (start 69.16 99.75) (end 69.16 108.64) (width 0.25) (layer "F.Cu") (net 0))
 (segment (start 99.858 91.707) (end 99.858 101.033) (width 0.15) (layer "F.Cu") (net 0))
 (segment (start 94.814 100.997) (end 94.56 101.251) (width 0.15) (layer "F.Cu") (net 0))
 (segment (start 97.1 88.551) (end 99.64 86.011) (width 0.15) (layer "F.Cu") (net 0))
 (segment (start 96.592 89.948) (end 103.323 89.948) (width 0.15) (layer "F.Cu") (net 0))
 (segment (start 57.73 99.75) (end 69.16 99.75) (width 0.25) (layer "F.Cu") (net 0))
 (segment (start 99.64 89.44) (end 101.291 89.44) (width 0.15) (layer "F.Cu") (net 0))
 (segment (start 100.529 99.6) (end 102.18 101.251) (width 0.15) (layer "F.Cu") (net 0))
 (segment (start 108.963 95.207) (end 109.8 96.044) (width 0.15) (layer "F.Cu") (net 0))
 (segment (start 45.03 99.75) (end 45.03 56.57) (width 0.25) (layer "F.Cu") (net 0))
 (segment (start 92.147 86.138) (end 92.02 86.011) (width 0.15) (layer "F.Cu") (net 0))
 (segment (start 36.14 37.52) (end 60.27 37.52) (width 0.25) (layer "F.Cu") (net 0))
 (segment (start 106.752 96.552) (end 107.26 97.06) (width 0.15) (layer "F.Cu") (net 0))
 (segment (start 96.846 90.456) (end 105.355 90.456) (width 0.15) (layer "F.Cu") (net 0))
 (segment (start 93.858 89.373) (end 93.163 88.678) (width 0.15) (layer "F.Cu") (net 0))
 (segment (start 117.42 80.7) (end 117.42 83.24) (width 0.2) (layer "F.Cu") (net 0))
 (segment (start 100.91 96.552) (end 106.752 96.552) (width 0.15) (layer "F.Cu") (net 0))
 (segment (start 95.458 89.177) (end 95.576 89.059) (width 0.15) (layer "F.Cu") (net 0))
 (segment (start 92.02 99.854) (end 92.02 101.251) (width 0.15) (layer "F.Cu") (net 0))
 (segment (start 109.8 103.56) (end 112.34 106.1) (width 0.2) (layer "F.Cu") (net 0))
 (segment (start 99.458 95.718) (end 96.973 98.203) (width 0.15) (layer "F.Cu") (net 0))
 (segment (start 107.26 108.64) (end 107.26 101.251) (width 0.2) (layer "F.Cu") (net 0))
 (segment (start 46.3 116.26) (end 112.34 116.26) (width 0.25) (layer "F.Cu") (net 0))
 (segment (start 43.76 68) (end 36.14 68) (width 0.25) (layer "F.Cu") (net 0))
 (segment (start 94.56 78.16) (end 94.56 86.011) (width 0.2) (layer "F.Cu") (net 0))
 (segment (start 94.658 87.691) (end 94.814 87.535) (width 0.15) (layer "F.Cu") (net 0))
 (segment (start 86.94 98.838) (end 86.94 101.251) (width 0.15) (layer "F.Cu") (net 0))
 (segment (start 95.058 88.942) (end 95.449 88.551) (width 0.15) (layer "F.Cu") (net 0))
 (segment (start 114.3 60.96) (end 112.34 62.92) (width 0.25) (layer "F.Cu") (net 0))
 (segment (start 71.7 75.62) (end 74.24 78.16) (width 0.2) (layer "F.Cu") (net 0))
 (segment (start 65.06 43.58) (end 64.08 42.6) (width 0.25) (layer "F.Cu") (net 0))
 (segment (start 100.258 93.36) (end 100.529 93.631) (width 0.15) (layer "F.Cu") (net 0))
 (segment (start 99.458 91.707) (end 99.458 95.718) (width 0.15) (layer "F.Cu") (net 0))
 (segment (start 83.13 97.187) (end 81.86 98.457) (width 0.15) (layer "F.Cu") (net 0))
 (segment (start 90.258 93.707) (end 91.258 92.707) (width 0.15) (layer "F.Cu") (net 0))
 (segment (start 100.529 98.33) (end 100.529 99.6) (width 0.15) (layer "F.Cu") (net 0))
 (segment (start 101.291 89.44) (end 104.72 86.011) (width 0.15) (layer "F.Cu") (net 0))
 (segment (start 87.321 89.186) (end 87.321 86.392) (width 0.15) (layer "F.Cu") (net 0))
 (segment (start 41.22 42.6) (end 36.14 37.52) (width 0.25) (layer "F.Cu") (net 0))
 (segment (start 74.24 78.16) (end 94.56 78.16) (width 0.2) (layer "F.Cu") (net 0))
 (segment (start 109.8 96.044) (end 109.8 101.251) (width 0.15) (layer "F.Cu") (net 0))
 (segment (start 109.8 101.251) (end 109.8 103.56) (width 0.2) (layer "F.Cu") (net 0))
 (segment (start 97.1 80.7) (end 97.1 86.011) (width 0.25) (layer "F.Cu") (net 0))
 (segment (start 104.14 37.52) (end 114.3 47.68) (width 0.25) (layer "F.Cu") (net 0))
 (segment (start 81.86 98.457) (end 81.86 101.251) (width 0.15) (layer "F.Cu") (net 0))
 (segment (start 93.458 91.707) (end 93.458 89.567) (width 0.15) (layer "F.Cu") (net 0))
 (segment (start 101.758 94.607) (end 101.758 95.207) (width 0.15) (layer "F.Cu") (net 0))
 (segment (start 114.88 73.08) (end 117.42 75.62) (width 0.25) (layer "F.Cu") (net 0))
 (segment (start 112.34 116.26) (end 117.42 116.26) (width 0.25) (layer "F.Cu") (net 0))
 (segment (start 87.321 86.392) (end 86.94 86.011) (width 0.15) (layer "F.Cu") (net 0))
 (segment (start 97.458 91.707) (end 97.458 93.4) (width 0.15) (layer "F.Cu") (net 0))
 (segment (start 94.258 91.707) (end 94.258 86.313) (width 0.15) (layer "F.Cu") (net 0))
 (segment (start 96.973 98.203) (end 96.973 101.124) (width 0.15) (layer "F.Cu") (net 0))
 (segment (start 107.26 108.64) (end 114.3 108.64) (width 0.25) (layer "F.Cu") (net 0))
 (segment (start 92.531 89.948) (end 86.686 89.948) (width 0.15) (layer "F.Cu") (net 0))
 (segment (start 45.03 99.75) (end 45.03 114.99) (width 0.25) (layer "F.Cu") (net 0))
 (segment (start 65.06 62.92) (end 65.06 43.58) (width 0.25) (layer "F.Cu") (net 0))
 (segment (start 64.52 62.92) (end 97.1 62.92) (width 0.25) (layer "F.Cu") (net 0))
 (segment (start 62.81 75.62) (end 71.7 75.62) (width 0.25) (layer "F.Cu") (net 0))
 (segment (start 85.162 97.695) (end 84.4 98.457) (width 0.15) (layer "F.Cu") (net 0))
 (segment (start 86.686 88.297) (end 84.4 86.011) (width 0.15) (layer "F.Cu") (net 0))
 (segment (start 97.858 91.707) (end 97.858 93.762) (width 0.15) (layer "F.Cu") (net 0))
 (segment (start 95.058 91.707) (end 95.058 88.942) (width 0.15) (layer "F.Cu") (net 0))
 (segment (start 45.03 114.99) (end 46.3 116.26) (width 0.25) (layer "F.Cu") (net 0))
 (via (at 43.76 68) (size 0.6) (drill 0.3) (layers "F.Cu" "B.Cu") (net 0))
 (via (at 46.3 68) (size 0.6) (drill 0.3) (layers "F.Cu" "B.Cu") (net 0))
 (via (at 100.529 93.631) (size 0.61) (drill 0.305) (layers "F.Cu" "B.Cu") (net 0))
 (via (at 46.3 65.46) (size 0.6) (drill 0.3) (layers "F.Cu" "B.Cu") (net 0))
 (via (at 100.529 98.33) (size 0.61) (drill 0.305) (layers "F.Cu" "B.Cu") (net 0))
 (via (at 97.1 80.7) (size 0.6) (drill 0.3) (layers "F.Cu" "B.Cu") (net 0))
 (via (at 104.72 99.473) (size 0.61) (drill 0.305) (layers "F.Cu" "B.Cu") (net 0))
 (via (at 97.1 75.62) (size 0.6) (drill 0.3) (layers "F.Cu" "B.Cu") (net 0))
 (via (at 93.29 94.012) (size 0.61) (drill 0.305) (layers "F.Cu" "B.Cu") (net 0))
 (via (at 112.34 106.1) (size 0.6) (drill 0.3) (layers "F.Cu" "B.Cu") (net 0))
 (via (at 112.34 111.18) (size 0.6) (drill 0.3) (layers "F.Cu" "B.Cu") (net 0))
 (via (at 43.76 65.46) (size 0.6) (drill 0.3) (layers "F.Cu" "B.Cu") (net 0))
 (segment (start 100.529 98.33) (end 100.529 93.631) (width 0.15) (layer "B.Cu") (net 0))
 (segment (start 43.76 65.46) (end 46.3 65.46) (width 0.25) (layer "B.Cu") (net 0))
 (segment (start 46.3 68) (end 43.76 68) (width 0.25) (layer "B.Cu") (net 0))
 (segment (start 91.258 92.107) (end 91.258 89.313) (width 0.15) (layer "B.Cu") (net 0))
 (segment (start 112.34 106.1) (end 112.34 111.18) (width 0.25) (layer "B.Cu") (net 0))
 (segment (start 94.179 99.473) (end 104.72 99.473) (width 0.15) (layer "B.Cu") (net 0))
 (segment (start 101.926 89.059) (end 101.758 89.227) (width 0.15) (layer "B.Cu") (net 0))
 (segment (start 97.1 75.62) (end 97.1 80.7) (width 0.25) (layer "B.Cu") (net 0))
 (segment (start 100.91 88.043) (end 101.926 89.059) (width 0.15) (layer "B.Cu") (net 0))
 (segment (start 93.29 94.012) (end 93.29 98.584) (width 0.15) (layer "B.Cu") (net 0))
 (segment (start 92.528 88.043) (end 100.91 88.043) (width 0.15) (layer "B.Cu") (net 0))
 (segment (start 91.258 89.313) (end 92.528 88.043) (width 0.15) (layer "B.Cu") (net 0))
 (segment (start 101.758 89.227) (end 101.758 92.107) (width 0.15) (layer "B.Cu") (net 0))
 (segment (start 93.29 98.584) (end 94.179 99.473) (width 0.15) (layer "B.Cu") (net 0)))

